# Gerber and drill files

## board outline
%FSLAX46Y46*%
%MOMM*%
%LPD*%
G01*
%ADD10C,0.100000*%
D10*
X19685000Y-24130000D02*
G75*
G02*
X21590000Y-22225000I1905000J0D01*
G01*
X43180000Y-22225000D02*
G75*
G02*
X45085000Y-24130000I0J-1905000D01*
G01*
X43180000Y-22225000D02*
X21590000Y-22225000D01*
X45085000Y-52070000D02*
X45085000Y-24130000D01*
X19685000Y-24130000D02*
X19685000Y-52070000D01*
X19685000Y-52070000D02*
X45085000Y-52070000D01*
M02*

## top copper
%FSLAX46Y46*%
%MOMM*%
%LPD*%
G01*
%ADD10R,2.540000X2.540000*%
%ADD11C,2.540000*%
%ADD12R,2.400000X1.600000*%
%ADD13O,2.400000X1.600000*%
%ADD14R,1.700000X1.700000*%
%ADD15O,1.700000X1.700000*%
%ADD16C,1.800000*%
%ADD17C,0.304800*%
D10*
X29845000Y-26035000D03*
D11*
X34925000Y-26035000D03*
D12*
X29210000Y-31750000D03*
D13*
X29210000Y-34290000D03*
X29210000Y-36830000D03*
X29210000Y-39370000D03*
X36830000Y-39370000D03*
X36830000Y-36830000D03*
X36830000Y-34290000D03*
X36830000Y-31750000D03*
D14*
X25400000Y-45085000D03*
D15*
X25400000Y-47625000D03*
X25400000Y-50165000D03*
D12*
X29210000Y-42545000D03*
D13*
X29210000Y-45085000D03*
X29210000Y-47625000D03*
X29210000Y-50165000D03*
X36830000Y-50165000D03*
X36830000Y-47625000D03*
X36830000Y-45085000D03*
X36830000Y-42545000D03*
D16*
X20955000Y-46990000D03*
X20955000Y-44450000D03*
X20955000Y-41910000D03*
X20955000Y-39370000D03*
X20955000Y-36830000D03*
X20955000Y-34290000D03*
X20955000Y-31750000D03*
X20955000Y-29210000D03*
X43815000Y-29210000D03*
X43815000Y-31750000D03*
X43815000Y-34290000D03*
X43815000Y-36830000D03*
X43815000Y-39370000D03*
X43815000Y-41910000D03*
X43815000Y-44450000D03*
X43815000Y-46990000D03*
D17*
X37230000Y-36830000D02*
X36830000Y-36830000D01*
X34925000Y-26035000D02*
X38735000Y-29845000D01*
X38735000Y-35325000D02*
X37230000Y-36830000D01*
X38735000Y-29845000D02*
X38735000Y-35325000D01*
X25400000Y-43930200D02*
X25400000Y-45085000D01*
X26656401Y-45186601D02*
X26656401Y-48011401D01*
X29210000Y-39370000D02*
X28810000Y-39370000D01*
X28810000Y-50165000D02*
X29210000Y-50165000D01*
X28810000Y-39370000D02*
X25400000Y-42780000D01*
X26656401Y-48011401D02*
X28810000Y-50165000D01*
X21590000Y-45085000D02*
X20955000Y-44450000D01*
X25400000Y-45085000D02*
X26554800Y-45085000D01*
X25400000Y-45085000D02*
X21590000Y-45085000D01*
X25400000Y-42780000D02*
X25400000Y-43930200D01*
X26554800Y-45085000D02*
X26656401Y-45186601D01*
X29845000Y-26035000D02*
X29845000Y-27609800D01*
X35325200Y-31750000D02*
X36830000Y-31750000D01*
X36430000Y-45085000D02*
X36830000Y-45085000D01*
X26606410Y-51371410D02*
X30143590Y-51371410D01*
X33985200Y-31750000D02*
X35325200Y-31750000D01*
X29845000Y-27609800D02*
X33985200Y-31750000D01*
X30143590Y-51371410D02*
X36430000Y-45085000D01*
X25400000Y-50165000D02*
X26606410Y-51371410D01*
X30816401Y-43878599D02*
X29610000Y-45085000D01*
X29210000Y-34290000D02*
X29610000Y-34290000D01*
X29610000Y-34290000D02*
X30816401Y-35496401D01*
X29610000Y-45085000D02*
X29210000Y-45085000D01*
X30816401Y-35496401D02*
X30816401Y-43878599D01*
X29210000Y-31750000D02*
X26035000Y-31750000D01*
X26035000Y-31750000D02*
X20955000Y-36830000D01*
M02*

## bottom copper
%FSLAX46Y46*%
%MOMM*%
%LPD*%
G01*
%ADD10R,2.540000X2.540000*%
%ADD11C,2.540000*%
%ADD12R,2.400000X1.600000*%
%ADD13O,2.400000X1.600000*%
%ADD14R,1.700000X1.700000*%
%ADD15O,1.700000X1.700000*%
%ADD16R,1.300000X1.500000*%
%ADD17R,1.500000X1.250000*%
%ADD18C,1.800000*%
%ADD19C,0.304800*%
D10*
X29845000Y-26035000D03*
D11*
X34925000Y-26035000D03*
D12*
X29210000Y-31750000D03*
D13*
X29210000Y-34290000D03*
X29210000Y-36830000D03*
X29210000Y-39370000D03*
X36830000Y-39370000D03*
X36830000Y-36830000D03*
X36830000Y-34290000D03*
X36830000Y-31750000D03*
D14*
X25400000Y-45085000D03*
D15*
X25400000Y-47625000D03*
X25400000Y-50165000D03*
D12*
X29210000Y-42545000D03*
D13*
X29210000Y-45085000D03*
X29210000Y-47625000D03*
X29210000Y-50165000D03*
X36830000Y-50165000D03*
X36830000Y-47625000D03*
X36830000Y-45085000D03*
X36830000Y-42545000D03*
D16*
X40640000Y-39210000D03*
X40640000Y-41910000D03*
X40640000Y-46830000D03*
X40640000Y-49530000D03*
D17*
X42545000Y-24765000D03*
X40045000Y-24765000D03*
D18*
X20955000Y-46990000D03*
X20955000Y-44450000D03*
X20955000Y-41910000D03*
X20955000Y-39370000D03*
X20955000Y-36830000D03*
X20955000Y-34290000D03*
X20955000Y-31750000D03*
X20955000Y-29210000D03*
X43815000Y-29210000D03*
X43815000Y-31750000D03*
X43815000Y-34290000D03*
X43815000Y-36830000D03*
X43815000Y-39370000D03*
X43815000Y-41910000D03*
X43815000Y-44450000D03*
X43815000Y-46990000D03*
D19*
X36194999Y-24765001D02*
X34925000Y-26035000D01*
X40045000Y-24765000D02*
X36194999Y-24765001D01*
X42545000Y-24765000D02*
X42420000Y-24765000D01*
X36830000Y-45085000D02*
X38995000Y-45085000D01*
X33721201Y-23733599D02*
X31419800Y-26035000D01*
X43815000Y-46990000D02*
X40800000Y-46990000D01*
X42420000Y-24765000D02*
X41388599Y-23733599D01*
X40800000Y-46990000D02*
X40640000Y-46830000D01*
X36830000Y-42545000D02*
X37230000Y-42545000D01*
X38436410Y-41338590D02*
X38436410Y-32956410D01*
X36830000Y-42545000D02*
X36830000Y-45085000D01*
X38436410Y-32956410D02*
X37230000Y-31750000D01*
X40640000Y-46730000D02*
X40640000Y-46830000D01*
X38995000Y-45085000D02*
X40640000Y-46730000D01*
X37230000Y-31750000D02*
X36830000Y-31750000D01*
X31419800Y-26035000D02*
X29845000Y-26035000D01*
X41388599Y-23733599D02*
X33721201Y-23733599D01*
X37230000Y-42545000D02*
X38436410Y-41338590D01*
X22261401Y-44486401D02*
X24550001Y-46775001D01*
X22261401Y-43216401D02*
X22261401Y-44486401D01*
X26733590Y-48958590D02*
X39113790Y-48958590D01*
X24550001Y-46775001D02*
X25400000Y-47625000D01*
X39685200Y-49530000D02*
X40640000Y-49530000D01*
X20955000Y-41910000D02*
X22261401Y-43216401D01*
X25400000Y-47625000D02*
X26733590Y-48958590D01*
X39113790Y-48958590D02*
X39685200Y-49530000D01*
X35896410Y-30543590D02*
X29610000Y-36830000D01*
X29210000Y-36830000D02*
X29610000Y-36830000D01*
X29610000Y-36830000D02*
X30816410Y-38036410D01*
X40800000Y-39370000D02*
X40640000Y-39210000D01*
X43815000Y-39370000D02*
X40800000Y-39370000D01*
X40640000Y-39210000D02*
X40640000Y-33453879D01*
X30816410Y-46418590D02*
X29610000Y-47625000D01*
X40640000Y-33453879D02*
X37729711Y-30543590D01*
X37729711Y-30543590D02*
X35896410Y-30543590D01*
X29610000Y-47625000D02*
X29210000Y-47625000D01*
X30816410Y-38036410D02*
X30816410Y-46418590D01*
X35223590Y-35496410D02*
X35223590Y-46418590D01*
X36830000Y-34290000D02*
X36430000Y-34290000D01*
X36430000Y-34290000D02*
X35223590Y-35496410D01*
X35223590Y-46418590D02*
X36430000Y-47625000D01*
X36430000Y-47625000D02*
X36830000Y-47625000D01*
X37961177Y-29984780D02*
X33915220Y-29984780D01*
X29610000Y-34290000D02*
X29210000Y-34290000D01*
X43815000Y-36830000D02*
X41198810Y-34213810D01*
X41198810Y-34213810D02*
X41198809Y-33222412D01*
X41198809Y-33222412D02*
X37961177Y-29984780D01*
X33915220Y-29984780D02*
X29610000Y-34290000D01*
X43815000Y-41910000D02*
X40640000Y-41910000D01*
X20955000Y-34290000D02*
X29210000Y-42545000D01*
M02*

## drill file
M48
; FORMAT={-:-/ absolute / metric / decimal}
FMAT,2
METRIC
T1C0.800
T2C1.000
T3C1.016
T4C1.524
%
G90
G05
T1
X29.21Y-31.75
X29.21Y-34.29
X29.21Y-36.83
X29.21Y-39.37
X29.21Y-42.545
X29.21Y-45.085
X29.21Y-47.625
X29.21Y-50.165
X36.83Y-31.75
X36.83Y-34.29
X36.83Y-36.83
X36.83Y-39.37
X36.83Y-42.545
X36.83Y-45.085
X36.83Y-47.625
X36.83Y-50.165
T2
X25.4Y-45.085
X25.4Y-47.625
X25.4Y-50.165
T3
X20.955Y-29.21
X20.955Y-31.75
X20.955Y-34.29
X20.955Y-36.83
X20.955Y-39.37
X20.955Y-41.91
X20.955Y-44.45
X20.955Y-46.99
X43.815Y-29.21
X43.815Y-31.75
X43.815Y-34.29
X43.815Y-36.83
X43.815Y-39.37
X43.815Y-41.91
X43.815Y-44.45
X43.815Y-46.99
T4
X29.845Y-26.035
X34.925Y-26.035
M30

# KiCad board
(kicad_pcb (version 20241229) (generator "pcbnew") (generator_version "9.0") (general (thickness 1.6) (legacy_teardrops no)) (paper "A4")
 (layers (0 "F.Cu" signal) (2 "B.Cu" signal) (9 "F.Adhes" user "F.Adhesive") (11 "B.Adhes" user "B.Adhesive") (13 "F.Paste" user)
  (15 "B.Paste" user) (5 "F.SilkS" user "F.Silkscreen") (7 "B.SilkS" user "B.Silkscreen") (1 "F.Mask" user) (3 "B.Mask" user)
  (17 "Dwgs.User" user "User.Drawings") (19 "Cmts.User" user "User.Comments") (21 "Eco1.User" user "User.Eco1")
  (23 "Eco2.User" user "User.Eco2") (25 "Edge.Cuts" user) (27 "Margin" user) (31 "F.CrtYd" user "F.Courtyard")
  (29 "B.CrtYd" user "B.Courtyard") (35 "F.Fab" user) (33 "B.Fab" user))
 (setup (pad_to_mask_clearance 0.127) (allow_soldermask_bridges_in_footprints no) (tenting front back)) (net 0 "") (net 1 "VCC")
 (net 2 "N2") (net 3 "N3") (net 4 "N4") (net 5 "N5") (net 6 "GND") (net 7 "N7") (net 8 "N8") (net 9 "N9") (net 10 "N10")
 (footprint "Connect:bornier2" (layer "F.Cu") (at 32.385 26.035)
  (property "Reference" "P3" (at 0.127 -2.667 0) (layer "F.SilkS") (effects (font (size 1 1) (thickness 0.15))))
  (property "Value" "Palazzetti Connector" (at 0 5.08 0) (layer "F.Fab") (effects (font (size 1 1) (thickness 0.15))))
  (pad "1" thru_hole rect (at -2.54 0) (size 2.54 2.54) (drill 1.524) (layers "*.Cu" "*.Mask") (remove_unused_layers no) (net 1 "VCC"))
  (pad "2" thru_hole circle (at 2.54 0) (size 2.54 2.54) (drill 1.524) (layers "*.Cu" "*.Mask") (remove_unused_layers no) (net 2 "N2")))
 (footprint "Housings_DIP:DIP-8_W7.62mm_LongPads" (layer "F.Cu") (at 29.21 31.75)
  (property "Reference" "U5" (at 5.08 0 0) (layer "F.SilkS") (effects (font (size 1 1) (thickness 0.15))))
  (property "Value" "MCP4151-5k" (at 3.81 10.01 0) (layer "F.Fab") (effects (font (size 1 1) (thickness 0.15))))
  (pad "1" thru_hole rect (at 0 0) (size 2.4 1.6) (drill 0.8) (layers "*.Cu" "*.Mask") (remove_unused_layers no) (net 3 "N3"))
  (pad "2" thru_hole oval (at 0 2.54) (size 2.4 1.6) (drill 0.8) (layers "*.Cu" "*.Mask") (remove_unused_layers no) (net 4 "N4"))
  (pad "3" thru_hole oval (at 0 5.08) (size 2.4 1.6) (drill 0.8) (layers "*.Cu" "*.Mask") (remove_unused_layers no) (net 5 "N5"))
  (pad "4" thru_hole oval (at 0 7.62) (size 2.4 1.6) (drill 0.8) (layers "*.Cu" "*.Mask") (remove_unused_layers no) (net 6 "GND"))
  (pad "5" thru_hole oval (at 7.62 7.62) (size 2.4 1.6) (drill 0.8) (layers "*.Cu" "*.Mask") (remove_unused_layers no))
  (pad "6" thru_hole oval (at 7.62 5.08) (size 2.4 1.6) (drill 0.8) (layers "*.Cu" "*.Mask") (remove_unused_layers no) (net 2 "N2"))
  (pad "7" thru_hole oval (at 7.62 2.54) (size 2.4 1.6) (drill 0.8) (layers "*.Cu" "*.Mask") (remove_unused_layers no) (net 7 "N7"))
  (pad "8" thru_hole oval (at 7.62 0) (size 2.4 1.6) (drill 0.8) (layers "*.Cu" "*.Mask") (remove_unused_layers no) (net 1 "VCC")))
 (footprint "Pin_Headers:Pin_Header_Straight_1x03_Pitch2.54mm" (layer "F.Cu") (at 25.4 45.085)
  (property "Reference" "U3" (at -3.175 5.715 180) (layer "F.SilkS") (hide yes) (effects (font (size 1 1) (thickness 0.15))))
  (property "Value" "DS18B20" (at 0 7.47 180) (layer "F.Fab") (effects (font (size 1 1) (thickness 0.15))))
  (pad "1" thru_hole rect (at 0 0) (size 1.7 1.7) (drill 1) (layers "*.Cu" "*.Mask") (remove_unused_layers no) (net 6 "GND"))
  (pad "2" thru_hole oval (at 0 2.54) (size 1.7 1.7) (drill 1) (layers "*.Cu" "*.Mask") (remove_unused_layers no) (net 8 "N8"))
  (pad "3" thru_hole oval (at 0 5.08) (size 1.7 1.7) (drill 1) (layers "*.Cu" "*.Mask") (remove_unused_layers no) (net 1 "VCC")))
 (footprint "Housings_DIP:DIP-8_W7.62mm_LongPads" (layer "F.Cu") (at 29.21 42.545)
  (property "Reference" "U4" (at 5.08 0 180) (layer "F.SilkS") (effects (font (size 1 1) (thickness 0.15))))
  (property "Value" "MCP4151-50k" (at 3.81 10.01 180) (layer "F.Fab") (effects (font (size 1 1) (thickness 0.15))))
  (pad "1" thru_hole rect (at 0 0) (size 2.4 1.6) (drill 0.8) (layers "*.Cu" "*.Mask") (remove_unused_layers no) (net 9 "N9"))
  (pad "2" thru_hole oval (at 0 2.54) (size 2.4 1.6) (drill 0.8) (layers "*.Cu" "*.Mask") (remove_unused_layers no) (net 4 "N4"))
  (pad "3" thru_hole oval (at 0 5.08) (size 2.4 1.6) (drill 0.8) (layers "*.Cu" "*.Mask") (remove_unused_layers no) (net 5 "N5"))
  (pad "4" thru_hole oval (at 0 7.62) (size 2.4 1.6) (drill 0.8) (layers "*.Cu" "*.Mask") (remove_unused_layers no) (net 6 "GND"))
  (pad "5" thru_hole oval (at 7.62 7.62) (size 2.4 1.6) (drill 0.8) (layers "*.Cu" "*.Mask") (remove_unused_layers no))
  (pad "6" thru_hole oval (at 7.62 5.08) (size 2.4 1.6) (drill 0.8) (layers "*.Cu" "*.Mask") (remove_unused_layers no) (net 7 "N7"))
  (pad "7" thru_hole oval (at 7.62 2.54) (size 2.4 1.6) (drill 0.8) (layers "*.Cu" "*.Mask") (remove_unused_layers no) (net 1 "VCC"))
  (pad "8" thru_hole oval (at 7.62 0) (size 2.4 1.6) (drill 0.8) (layers "*.Cu" "*.Mask") (remove_unused_layers no) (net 1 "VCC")))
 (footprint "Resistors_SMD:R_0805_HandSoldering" (layer "B.Cu") (at 40.64 40.56 -90)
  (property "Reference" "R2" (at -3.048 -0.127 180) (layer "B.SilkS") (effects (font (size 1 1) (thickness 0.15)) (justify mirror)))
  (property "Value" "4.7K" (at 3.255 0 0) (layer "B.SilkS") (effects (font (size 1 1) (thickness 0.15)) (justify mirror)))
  (pad "1" smd rect (at -1.35 0 270) (size 1.5 1.3) (layers "B.Cu" "B.Mask" "B.Paste") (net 5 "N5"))
  (pad "2" smd rect (at 1.35 0 270) (size 1.5 1.3) (layers "B.Cu" "B.Mask" "B.Paste") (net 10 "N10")))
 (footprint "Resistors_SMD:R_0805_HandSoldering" (layer "B.Cu") (at 40.64 48.18 -90)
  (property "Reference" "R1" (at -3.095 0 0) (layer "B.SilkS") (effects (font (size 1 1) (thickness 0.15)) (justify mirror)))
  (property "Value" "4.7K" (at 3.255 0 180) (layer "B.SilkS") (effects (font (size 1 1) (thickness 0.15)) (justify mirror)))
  (pad "1" smd rect (at -1.35 0 270) (size 1.5 1.3) (layers "B.Cu" "B.Mask" "B.Paste") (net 1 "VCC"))
  (pad "2" smd rect (at 1.35 0 270) (size 1.5 1.3) (layers "B.Cu" "B.Mask" "B.Paste") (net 8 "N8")))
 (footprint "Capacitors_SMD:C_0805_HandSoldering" (layer "B.Cu") (at 41.295 24.765 180)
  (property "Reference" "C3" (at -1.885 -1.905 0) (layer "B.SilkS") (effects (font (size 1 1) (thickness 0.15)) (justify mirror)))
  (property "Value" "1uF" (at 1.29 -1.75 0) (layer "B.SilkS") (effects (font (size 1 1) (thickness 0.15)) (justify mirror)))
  (pad "1" smd rect (at -1.25 0 180) (size 1.5 1.25) (layers "B.Cu" "B.Mask" "B.Paste") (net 1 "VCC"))
  (pad "2" smd rect (at 1.25 0 180) (size 1.5 1.25) (layers "B.Cu" "B.Mask" "B.Paste") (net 2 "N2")))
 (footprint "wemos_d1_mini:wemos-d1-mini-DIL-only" (layer "B.Cu") (at 32.385 38.1 90)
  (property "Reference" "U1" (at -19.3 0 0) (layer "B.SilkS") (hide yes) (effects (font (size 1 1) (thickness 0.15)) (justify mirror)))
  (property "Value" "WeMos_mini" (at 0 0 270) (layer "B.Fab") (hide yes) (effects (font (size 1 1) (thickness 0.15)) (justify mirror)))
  (pad "1" thru_hole circle (at -8.89 -11.43 90) (size 1.8 1.8) (drill 1.016) (layers "*.Cu" "*.Mask") (remove_unused_layers no))
  (pad "2" thru_hole circle (at -6.35 -11.43 90) (size 1.8 1.8) (drill 1.016) (layers "*.Cu" "*.Mask") (remove_unused_layers no)
   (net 6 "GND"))
  (pad "3" thru_hole circle (at -3.81 -11.43 90) (size 1.8 1.8) (drill 1.016) (layers "*.Cu" "*.Mask") (remove_unused_layers no)
   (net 8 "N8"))
  (pad "4" thru_hole circle (at -1.27 -11.43 90) (size 1.8 1.8) (drill 1.016) (layers "*.Cu" "*.Mask") (remove_unused_layers no))
  (pad "5" thru_hole circle (at 1.27 -11.43 90) (size 1.8 1.8) (drill 1.016) (layers "*.Cu" "*.Mask") (remove_unused_layers no) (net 3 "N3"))
  (pad "6" thru_hole circle (at 3.81 -11.43 90) (size 1.8 1.8) (drill 1.016) (layers "*.Cu" "*.Mask") (remove_unused_layers no) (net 9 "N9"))
  (pad "7" thru_hole circle (at 6.35 -11.43 90) (size 1.8 1.8) (drill 1.016) (layers "*.Cu" "*.Mask") (remove_unused_layers no))
  (pad "8" thru_hole circle (at 8.89 -11.43 90) (size 1.8 1.8) (drill 1.016) (layers "*.Cu" "*.Mask") (remove_unused_layers no))
  (pad "9" thru_hole circle (at 8.89 11.43 90) (size 1.8 1.8) (drill 1.016) (layers "*.Cu" "*.Mask") (remove_unused_layers no))
  (pad "10" thru_hole circle (at 6.35 11.43 90) (size 1.8 1.8) (drill 1.016) (layers "*.Cu" "*.Mask") (remove_unused_layers no))
  (pad "11" thru_hole circle (at 3.81 11.43 90) (size 1.8 1.8) (drill 1.016) (layers "*.Cu" "*.Mask") (remove_unused_layers no))
  (pad "12" thru_hole circle (at 1.27 11.43 90) (size 1.8 1.8) (drill 1.016) (layers "*.Cu" "*.Mask") (remove_unused_layers no) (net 4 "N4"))
  (pad "13" thru_hole circle (at -1.27 11.43 90) (size 1.8 1.8) (drill 1.016) (layers "*.Cu" "*.Mask") (remove_unused_layers no)
   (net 5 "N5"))
  (pad "14" thru_hole circle (at -3.81 11.43 90) (size 1.8 1.8) (drill 1.016) (layers "*.Cu" "*.Mask") (remove_unused_layers no)
   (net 10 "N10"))
  (pad "15" thru_hole circle (at -6.35 11.43 90) (size 1.8 1.8) (drill 1.016) (layers "*.Cu" "*.Mask") (remove_unused_layers no))
  (pad "16" thru_hole circle (at -8.89 11.43 90) (size 1.8 1.8) (drill 1.016) (layers "*.Cu" "*.Mask") (remove_unused_layers no)
   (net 1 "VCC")))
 (gr_arc (start 19.685 24.13) (mid 20.242962 22.782962) (end 21.59 22.225) (stroke (width 0.1) (type solid)) (layer "Edge.Cuts"))
 (gr_arc (start 43.18 22.225) (mid 44.527038 22.782962) (end 45.085 24.13) (stroke (width 0.1) (type solid)) (layer "Edge.Cuts"))
 (gr_line (start 43.18 22.225) (end 21.59 22.225) (stroke (width 0.1) (type solid)) (layer "Edge.Cuts"))
 (gr_line (start 45.085 52.07) (end 45.085 24.13) (stroke (width 0.1) (type solid)) (layer "Edge.Cuts"))
 (gr_line (start 19.685 24.13) (end 19.685 52.07) (stroke (width 0.1) (type solid)) (layer "Edge.Cuts"))
 (gr_line (start 19.685 52.07) (end 45.085 52.07) (stroke (width 0.1) (type solid)) (layer "Edge.Cuts"))
 (segment (start 37.23 36.83) (end 36.83 36.83) (width 0.3048) (layer "F.Cu") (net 2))
 (segment (start 34.925 26.035) (end 38.735 29.845) (width 0.3048) (layer "F.Cu") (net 2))
 (segment (start 38.735 35.325) (end 37.23 36.83) (width 0.3048) (layer "F.Cu") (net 2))
 (segment (start 38.735 29.845) (end 38.735 35.325) (width 0.3048) (layer "F.Cu") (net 2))
 (segment (start 36.194999 24.765001) (end 34.925 26.035) (width 0.3048) (layer "B.Cu") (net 2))
 (segment (start 40.045 24.765) (end 36.194999 24.765001) (width 0.3048) (layer "B.Cu") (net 2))
 (segment (start 25.4 43.9302) (end 25.4 45.085) (width 0.3048) (layer "F.Cu") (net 6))
 (segment (start 26.656401 45.186601) (end 26.656401 48.011401) (width 0.3048) (layer "F.Cu") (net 6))
 (segment (start 29.21 39.37) (end 28.81 39.37) (width 0.3048) (layer "F.Cu") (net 6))
 (segment (start 28.81 50.165) (end 29.21 50.165) (width 0.3048) (layer "F.Cu") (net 6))
 (segment (start 28.81 39.37) (end 25.4 42.78) (width 0.3048) (layer "F.Cu") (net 6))
 (segment (start 26.656401 48.011401) (end 28.81 50.165) (width 0.3048) (layer "F.Cu") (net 6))
 (segment (start 21.59 45.085) (end 20.955 44.45) (width 0.3048) (layer "F.Cu") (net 6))
 (segment (start 25.4 45.085) (end 26.5548 45.085) (width 0.3048) (layer "F.Cu") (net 6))
 (segment (start 25.4 45.085) (end 21.59 45.085) (width 0.3048) (layer "F.Cu") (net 6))
 (segment (start 25.4 42.78) (end 25.4 43.9302) (width 0.3048) (layer "F.Cu") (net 6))
 (segment (start 26.5548 45.085) (end 26.656401 45.186601) (width 0.3048) (layer "F.Cu") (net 6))
 (segment (start 29.845 26.035) (end 29.845 27.6098) (width 0.3048) (layer "F.Cu") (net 1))
 (segment (start 35.3252 31.75) (end 36.83 31.75) (width 0.3048) (layer "F.Cu") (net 1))
 (segment (start 36.43 45.085) (end 36.83 45.085) (width 0.3048) (layer "F.Cu") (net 1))
 (segment (start 26.60641 51.37141) (end 30.14359 51.37141) (width 0.3048) (layer "F.Cu") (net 1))
 (segment (start 33.9852 31.75) (end 35.3252 31.75) (width 0.3048) (layer "F.Cu") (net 1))
 (segment (start 29.845 27.6098) (end 33.9852 31.75) (width 0.3048) (layer "F.Cu") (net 1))
 (segment (start 30.14359 51.37141) (end 36.43 45.085) (width 0.3048) (layer "F.Cu") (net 1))
 (segment (start 25.4 50.165) (end 26.60641 51.37141) (width 0.3048) (layer "F.Cu") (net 1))
 (segment (start 42.545 24.765) (end 42.42 24.765) (width 0.3048) (layer "B.Cu") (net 1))
 (segment (start 36.83 45.085) (end 38.995 45.085) (width 0.3048) (layer "B.Cu") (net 1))
 (segment (start 33.721201 23.733599) (end 31.4198 26.035) (width 0.3048) (layer "B.Cu") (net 1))
 (segment (start 43.815 46.99) (end 40.8 46.99) (width 0.3048) (layer "B.Cu") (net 1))
 (segment (start 42.42 24.765) (end 41.388599 23.733599) (width 0.3048) (layer "B.Cu") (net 1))
 (segment (start 40.8 46.99) (end 40.64 46.83) (width 0.3048) (layer "B.Cu") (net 1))
 (segment (start 36.83 42.545) (end 37.23 42.545) (width 0.3048) (layer "B.Cu") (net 1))
 (segment (start 38.43641 41.33859) (end 38.43641 32.95641) (width 0.3048) (layer "B.Cu") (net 1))
 (segment (start 36.83 42.545) (end 36.83 45.085) (width 0.3048) (layer "B.Cu") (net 1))
 (segment (start 38.43641 32.95641) (end 37.23 31.75) (width 0.3048) (layer "B.Cu") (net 1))
 (segment (start 40.64 46.73) (end 40.64 46.83) (width 0.3048) (layer "B.Cu") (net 1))
 (segment (start 38.995 45.085) (end 40.64 46.73) (width 0.3048) (layer "B.Cu") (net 1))
 (segment (start 37.23 31.75) (end 36.83 31.75) (width 0.3048) (layer "B.Cu") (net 1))
 (segment (start 31.4198 26.035) (end 29.845 26.035) (width 0.3048) (layer "B.Cu") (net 1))
 (segment (start 41.388599 23.733599) (end 33.721201 23.733599) (width 0.3048) (layer "B.Cu") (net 1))
 (segment (start 37.23 42.545) (end 38.43641 41.33859) (width 0.3048) (layer "B.Cu") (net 1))
 (segment (start 22.261401 44.486401) (end 24.550001 46.775001) (width 0.3048) (layer "B.Cu") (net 8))
 (segment (start 22.261401 43.216401) (end 22.261401 44.486401) (width 0.3048) (layer "B.Cu") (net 8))
 (segment (start 26.73359 48.95859) (end 39.11379 48.95859) (width 0.3048) (layer "B.Cu") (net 8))
 (segment (start 24.550001 46.775001) (end 25.4 47.625) (width 0.3048) (layer "B.Cu") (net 8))
 (segment (start 39.6852 49.53) (end 40.64 49.53) (width 0.3048) (layer "B.Cu") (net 8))
 (segment (start 20.955 41.91) (end 22.261401 43.216401) (width 0.3048) (layer "B.Cu") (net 8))
 (segment (start 25.4 47.625) (end 26.73359 48.95859) (width 0.3048) (layer "B.Cu") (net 8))
 (segment (start 39.11379 48.95859) (end 39.6852 49.53) (width 0.3048) (layer "B.Cu") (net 8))
 (segment (start 35.89641 30.54359) (end 29.61 36.83) (width 0.3048) (layer "B.Cu") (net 5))
 (segment (start 29.21 36.83) (end 29.61 36.83) (width 0.3048) (layer "B.Cu") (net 5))
 (segment (start 29.61 36.83) (end 30.81641 38.03641) (width 0.3048) (layer "B.Cu") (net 5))
 (segment (start 40.8 39.37) (end 40.64 39.21) (width 0.3048) (layer "B.Cu") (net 5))
 (segment (start 43.815 39.37) (end 40.8 39.37) (width 0.3048) (layer "B.Cu") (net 5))
 (segment (start 40.64 39.21) (end 40.64 33.453879) (width 0.3048) (layer "B.Cu") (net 5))
 (segment (start 30.81641 46.41859) (end 29.61 47.625) (width 0.3048) (layer "B.Cu") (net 5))
 (segment (start 40.64 33.453879) (end 37.729711 30.54359) (width 0.3048) (layer "B.Cu") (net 5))
 (segment (start 37.729711 30.54359) (end 35.89641 30.54359) (width 0.3048) (layer "B.Cu") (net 5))
 (segment (start 29.61 47.625) (end 29.21 47.625) (width 0.3048) (layer "B.Cu") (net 5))
 (segment (start 30.81641 38.03641) (end 30.81641 46.41859) (width 0.3048) (layer "B.Cu") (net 5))
 (segment (start 35.22359 35.49641) (end 35.22359 46.41859) (width 0.3048) (layer "B.Cu") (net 7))
 (segment (start 36.83 34.29) (end 36.43 34.29) (width 0.3048) (layer "B.Cu") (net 7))
 (segment (start 36.43 34.29) (end 35.22359 35.49641) (width 0.3048) (layer "B.Cu") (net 7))
 (segment (start 35.22359 46.41859) (end 36.43 47.625) (width 0.3048) (layer "B.Cu") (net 7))
 (segment (start 36.43 47.625) (end 36.83 47.625) (width 0.3048) (layer "B.Cu") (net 7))
 (segment (start 30.816401 43.878599) (end 29.61 45.085) (width 0.3048) (layer "F.Cu") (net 4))
 (segment (start 29.21 34.29) (end 29.61 34.29) (width 0.3048) (layer "F.Cu") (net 4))
 (segment (start 29.61 34.29) (end 30.816401 35.496401) (width 0.3048) (layer "F.Cu") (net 4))
 (segment (start 29.61 45.085) (end 29.21 45.085) (width 0.3048) (layer "F.Cu") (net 4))
 (segment (start 30.816401 35.496401) (end 30.816401 43.878599) (width 0.3048) (layer "F.Cu") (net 4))
 (segment (start 37.961177 29.98478) (end 33.91522 29.98478) (width 0.3048) (layer "B.Cu") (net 4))
 (segment (start 29.61 34.29) (end 29.21 34.29) (width 0.3048) (layer "B.Cu") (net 4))
 (segment (start 43.815 36.83) (end 41.19881 34.21381) (width 0.3048) (layer "B.Cu") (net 4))
 (segment (start 41.19881 34.21381) (end 41.198809 33.222412) (width 0.3048) (layer "B.Cu") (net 4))
 (segment (start 41.198809 33.222412) (end 37.961177 29.98478) (width 0.3048) (layer "B.Cu") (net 4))
 (segment (start 33.91522 29.98478) (end 29.61 34.29) (width 0.3048) (layer "B.Cu") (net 4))
 (segment (start 43.815 41.91) (end 40.64 41.91) (width 0.3048) (layer "B.Cu") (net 10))
 (segment (start 29.21 31.75) (end 26.035 31.75) (width 0.3048) (layer "F.Cu") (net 3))
 (segment (start 26.035 31.75) (end 20.955 36.83) (width 0.3048) (layer "F.Cu") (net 3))
 (segment (start 20.955 34.29) (end 29.21 42.545) (width 0.3048) (layer "B.Cu") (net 9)))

